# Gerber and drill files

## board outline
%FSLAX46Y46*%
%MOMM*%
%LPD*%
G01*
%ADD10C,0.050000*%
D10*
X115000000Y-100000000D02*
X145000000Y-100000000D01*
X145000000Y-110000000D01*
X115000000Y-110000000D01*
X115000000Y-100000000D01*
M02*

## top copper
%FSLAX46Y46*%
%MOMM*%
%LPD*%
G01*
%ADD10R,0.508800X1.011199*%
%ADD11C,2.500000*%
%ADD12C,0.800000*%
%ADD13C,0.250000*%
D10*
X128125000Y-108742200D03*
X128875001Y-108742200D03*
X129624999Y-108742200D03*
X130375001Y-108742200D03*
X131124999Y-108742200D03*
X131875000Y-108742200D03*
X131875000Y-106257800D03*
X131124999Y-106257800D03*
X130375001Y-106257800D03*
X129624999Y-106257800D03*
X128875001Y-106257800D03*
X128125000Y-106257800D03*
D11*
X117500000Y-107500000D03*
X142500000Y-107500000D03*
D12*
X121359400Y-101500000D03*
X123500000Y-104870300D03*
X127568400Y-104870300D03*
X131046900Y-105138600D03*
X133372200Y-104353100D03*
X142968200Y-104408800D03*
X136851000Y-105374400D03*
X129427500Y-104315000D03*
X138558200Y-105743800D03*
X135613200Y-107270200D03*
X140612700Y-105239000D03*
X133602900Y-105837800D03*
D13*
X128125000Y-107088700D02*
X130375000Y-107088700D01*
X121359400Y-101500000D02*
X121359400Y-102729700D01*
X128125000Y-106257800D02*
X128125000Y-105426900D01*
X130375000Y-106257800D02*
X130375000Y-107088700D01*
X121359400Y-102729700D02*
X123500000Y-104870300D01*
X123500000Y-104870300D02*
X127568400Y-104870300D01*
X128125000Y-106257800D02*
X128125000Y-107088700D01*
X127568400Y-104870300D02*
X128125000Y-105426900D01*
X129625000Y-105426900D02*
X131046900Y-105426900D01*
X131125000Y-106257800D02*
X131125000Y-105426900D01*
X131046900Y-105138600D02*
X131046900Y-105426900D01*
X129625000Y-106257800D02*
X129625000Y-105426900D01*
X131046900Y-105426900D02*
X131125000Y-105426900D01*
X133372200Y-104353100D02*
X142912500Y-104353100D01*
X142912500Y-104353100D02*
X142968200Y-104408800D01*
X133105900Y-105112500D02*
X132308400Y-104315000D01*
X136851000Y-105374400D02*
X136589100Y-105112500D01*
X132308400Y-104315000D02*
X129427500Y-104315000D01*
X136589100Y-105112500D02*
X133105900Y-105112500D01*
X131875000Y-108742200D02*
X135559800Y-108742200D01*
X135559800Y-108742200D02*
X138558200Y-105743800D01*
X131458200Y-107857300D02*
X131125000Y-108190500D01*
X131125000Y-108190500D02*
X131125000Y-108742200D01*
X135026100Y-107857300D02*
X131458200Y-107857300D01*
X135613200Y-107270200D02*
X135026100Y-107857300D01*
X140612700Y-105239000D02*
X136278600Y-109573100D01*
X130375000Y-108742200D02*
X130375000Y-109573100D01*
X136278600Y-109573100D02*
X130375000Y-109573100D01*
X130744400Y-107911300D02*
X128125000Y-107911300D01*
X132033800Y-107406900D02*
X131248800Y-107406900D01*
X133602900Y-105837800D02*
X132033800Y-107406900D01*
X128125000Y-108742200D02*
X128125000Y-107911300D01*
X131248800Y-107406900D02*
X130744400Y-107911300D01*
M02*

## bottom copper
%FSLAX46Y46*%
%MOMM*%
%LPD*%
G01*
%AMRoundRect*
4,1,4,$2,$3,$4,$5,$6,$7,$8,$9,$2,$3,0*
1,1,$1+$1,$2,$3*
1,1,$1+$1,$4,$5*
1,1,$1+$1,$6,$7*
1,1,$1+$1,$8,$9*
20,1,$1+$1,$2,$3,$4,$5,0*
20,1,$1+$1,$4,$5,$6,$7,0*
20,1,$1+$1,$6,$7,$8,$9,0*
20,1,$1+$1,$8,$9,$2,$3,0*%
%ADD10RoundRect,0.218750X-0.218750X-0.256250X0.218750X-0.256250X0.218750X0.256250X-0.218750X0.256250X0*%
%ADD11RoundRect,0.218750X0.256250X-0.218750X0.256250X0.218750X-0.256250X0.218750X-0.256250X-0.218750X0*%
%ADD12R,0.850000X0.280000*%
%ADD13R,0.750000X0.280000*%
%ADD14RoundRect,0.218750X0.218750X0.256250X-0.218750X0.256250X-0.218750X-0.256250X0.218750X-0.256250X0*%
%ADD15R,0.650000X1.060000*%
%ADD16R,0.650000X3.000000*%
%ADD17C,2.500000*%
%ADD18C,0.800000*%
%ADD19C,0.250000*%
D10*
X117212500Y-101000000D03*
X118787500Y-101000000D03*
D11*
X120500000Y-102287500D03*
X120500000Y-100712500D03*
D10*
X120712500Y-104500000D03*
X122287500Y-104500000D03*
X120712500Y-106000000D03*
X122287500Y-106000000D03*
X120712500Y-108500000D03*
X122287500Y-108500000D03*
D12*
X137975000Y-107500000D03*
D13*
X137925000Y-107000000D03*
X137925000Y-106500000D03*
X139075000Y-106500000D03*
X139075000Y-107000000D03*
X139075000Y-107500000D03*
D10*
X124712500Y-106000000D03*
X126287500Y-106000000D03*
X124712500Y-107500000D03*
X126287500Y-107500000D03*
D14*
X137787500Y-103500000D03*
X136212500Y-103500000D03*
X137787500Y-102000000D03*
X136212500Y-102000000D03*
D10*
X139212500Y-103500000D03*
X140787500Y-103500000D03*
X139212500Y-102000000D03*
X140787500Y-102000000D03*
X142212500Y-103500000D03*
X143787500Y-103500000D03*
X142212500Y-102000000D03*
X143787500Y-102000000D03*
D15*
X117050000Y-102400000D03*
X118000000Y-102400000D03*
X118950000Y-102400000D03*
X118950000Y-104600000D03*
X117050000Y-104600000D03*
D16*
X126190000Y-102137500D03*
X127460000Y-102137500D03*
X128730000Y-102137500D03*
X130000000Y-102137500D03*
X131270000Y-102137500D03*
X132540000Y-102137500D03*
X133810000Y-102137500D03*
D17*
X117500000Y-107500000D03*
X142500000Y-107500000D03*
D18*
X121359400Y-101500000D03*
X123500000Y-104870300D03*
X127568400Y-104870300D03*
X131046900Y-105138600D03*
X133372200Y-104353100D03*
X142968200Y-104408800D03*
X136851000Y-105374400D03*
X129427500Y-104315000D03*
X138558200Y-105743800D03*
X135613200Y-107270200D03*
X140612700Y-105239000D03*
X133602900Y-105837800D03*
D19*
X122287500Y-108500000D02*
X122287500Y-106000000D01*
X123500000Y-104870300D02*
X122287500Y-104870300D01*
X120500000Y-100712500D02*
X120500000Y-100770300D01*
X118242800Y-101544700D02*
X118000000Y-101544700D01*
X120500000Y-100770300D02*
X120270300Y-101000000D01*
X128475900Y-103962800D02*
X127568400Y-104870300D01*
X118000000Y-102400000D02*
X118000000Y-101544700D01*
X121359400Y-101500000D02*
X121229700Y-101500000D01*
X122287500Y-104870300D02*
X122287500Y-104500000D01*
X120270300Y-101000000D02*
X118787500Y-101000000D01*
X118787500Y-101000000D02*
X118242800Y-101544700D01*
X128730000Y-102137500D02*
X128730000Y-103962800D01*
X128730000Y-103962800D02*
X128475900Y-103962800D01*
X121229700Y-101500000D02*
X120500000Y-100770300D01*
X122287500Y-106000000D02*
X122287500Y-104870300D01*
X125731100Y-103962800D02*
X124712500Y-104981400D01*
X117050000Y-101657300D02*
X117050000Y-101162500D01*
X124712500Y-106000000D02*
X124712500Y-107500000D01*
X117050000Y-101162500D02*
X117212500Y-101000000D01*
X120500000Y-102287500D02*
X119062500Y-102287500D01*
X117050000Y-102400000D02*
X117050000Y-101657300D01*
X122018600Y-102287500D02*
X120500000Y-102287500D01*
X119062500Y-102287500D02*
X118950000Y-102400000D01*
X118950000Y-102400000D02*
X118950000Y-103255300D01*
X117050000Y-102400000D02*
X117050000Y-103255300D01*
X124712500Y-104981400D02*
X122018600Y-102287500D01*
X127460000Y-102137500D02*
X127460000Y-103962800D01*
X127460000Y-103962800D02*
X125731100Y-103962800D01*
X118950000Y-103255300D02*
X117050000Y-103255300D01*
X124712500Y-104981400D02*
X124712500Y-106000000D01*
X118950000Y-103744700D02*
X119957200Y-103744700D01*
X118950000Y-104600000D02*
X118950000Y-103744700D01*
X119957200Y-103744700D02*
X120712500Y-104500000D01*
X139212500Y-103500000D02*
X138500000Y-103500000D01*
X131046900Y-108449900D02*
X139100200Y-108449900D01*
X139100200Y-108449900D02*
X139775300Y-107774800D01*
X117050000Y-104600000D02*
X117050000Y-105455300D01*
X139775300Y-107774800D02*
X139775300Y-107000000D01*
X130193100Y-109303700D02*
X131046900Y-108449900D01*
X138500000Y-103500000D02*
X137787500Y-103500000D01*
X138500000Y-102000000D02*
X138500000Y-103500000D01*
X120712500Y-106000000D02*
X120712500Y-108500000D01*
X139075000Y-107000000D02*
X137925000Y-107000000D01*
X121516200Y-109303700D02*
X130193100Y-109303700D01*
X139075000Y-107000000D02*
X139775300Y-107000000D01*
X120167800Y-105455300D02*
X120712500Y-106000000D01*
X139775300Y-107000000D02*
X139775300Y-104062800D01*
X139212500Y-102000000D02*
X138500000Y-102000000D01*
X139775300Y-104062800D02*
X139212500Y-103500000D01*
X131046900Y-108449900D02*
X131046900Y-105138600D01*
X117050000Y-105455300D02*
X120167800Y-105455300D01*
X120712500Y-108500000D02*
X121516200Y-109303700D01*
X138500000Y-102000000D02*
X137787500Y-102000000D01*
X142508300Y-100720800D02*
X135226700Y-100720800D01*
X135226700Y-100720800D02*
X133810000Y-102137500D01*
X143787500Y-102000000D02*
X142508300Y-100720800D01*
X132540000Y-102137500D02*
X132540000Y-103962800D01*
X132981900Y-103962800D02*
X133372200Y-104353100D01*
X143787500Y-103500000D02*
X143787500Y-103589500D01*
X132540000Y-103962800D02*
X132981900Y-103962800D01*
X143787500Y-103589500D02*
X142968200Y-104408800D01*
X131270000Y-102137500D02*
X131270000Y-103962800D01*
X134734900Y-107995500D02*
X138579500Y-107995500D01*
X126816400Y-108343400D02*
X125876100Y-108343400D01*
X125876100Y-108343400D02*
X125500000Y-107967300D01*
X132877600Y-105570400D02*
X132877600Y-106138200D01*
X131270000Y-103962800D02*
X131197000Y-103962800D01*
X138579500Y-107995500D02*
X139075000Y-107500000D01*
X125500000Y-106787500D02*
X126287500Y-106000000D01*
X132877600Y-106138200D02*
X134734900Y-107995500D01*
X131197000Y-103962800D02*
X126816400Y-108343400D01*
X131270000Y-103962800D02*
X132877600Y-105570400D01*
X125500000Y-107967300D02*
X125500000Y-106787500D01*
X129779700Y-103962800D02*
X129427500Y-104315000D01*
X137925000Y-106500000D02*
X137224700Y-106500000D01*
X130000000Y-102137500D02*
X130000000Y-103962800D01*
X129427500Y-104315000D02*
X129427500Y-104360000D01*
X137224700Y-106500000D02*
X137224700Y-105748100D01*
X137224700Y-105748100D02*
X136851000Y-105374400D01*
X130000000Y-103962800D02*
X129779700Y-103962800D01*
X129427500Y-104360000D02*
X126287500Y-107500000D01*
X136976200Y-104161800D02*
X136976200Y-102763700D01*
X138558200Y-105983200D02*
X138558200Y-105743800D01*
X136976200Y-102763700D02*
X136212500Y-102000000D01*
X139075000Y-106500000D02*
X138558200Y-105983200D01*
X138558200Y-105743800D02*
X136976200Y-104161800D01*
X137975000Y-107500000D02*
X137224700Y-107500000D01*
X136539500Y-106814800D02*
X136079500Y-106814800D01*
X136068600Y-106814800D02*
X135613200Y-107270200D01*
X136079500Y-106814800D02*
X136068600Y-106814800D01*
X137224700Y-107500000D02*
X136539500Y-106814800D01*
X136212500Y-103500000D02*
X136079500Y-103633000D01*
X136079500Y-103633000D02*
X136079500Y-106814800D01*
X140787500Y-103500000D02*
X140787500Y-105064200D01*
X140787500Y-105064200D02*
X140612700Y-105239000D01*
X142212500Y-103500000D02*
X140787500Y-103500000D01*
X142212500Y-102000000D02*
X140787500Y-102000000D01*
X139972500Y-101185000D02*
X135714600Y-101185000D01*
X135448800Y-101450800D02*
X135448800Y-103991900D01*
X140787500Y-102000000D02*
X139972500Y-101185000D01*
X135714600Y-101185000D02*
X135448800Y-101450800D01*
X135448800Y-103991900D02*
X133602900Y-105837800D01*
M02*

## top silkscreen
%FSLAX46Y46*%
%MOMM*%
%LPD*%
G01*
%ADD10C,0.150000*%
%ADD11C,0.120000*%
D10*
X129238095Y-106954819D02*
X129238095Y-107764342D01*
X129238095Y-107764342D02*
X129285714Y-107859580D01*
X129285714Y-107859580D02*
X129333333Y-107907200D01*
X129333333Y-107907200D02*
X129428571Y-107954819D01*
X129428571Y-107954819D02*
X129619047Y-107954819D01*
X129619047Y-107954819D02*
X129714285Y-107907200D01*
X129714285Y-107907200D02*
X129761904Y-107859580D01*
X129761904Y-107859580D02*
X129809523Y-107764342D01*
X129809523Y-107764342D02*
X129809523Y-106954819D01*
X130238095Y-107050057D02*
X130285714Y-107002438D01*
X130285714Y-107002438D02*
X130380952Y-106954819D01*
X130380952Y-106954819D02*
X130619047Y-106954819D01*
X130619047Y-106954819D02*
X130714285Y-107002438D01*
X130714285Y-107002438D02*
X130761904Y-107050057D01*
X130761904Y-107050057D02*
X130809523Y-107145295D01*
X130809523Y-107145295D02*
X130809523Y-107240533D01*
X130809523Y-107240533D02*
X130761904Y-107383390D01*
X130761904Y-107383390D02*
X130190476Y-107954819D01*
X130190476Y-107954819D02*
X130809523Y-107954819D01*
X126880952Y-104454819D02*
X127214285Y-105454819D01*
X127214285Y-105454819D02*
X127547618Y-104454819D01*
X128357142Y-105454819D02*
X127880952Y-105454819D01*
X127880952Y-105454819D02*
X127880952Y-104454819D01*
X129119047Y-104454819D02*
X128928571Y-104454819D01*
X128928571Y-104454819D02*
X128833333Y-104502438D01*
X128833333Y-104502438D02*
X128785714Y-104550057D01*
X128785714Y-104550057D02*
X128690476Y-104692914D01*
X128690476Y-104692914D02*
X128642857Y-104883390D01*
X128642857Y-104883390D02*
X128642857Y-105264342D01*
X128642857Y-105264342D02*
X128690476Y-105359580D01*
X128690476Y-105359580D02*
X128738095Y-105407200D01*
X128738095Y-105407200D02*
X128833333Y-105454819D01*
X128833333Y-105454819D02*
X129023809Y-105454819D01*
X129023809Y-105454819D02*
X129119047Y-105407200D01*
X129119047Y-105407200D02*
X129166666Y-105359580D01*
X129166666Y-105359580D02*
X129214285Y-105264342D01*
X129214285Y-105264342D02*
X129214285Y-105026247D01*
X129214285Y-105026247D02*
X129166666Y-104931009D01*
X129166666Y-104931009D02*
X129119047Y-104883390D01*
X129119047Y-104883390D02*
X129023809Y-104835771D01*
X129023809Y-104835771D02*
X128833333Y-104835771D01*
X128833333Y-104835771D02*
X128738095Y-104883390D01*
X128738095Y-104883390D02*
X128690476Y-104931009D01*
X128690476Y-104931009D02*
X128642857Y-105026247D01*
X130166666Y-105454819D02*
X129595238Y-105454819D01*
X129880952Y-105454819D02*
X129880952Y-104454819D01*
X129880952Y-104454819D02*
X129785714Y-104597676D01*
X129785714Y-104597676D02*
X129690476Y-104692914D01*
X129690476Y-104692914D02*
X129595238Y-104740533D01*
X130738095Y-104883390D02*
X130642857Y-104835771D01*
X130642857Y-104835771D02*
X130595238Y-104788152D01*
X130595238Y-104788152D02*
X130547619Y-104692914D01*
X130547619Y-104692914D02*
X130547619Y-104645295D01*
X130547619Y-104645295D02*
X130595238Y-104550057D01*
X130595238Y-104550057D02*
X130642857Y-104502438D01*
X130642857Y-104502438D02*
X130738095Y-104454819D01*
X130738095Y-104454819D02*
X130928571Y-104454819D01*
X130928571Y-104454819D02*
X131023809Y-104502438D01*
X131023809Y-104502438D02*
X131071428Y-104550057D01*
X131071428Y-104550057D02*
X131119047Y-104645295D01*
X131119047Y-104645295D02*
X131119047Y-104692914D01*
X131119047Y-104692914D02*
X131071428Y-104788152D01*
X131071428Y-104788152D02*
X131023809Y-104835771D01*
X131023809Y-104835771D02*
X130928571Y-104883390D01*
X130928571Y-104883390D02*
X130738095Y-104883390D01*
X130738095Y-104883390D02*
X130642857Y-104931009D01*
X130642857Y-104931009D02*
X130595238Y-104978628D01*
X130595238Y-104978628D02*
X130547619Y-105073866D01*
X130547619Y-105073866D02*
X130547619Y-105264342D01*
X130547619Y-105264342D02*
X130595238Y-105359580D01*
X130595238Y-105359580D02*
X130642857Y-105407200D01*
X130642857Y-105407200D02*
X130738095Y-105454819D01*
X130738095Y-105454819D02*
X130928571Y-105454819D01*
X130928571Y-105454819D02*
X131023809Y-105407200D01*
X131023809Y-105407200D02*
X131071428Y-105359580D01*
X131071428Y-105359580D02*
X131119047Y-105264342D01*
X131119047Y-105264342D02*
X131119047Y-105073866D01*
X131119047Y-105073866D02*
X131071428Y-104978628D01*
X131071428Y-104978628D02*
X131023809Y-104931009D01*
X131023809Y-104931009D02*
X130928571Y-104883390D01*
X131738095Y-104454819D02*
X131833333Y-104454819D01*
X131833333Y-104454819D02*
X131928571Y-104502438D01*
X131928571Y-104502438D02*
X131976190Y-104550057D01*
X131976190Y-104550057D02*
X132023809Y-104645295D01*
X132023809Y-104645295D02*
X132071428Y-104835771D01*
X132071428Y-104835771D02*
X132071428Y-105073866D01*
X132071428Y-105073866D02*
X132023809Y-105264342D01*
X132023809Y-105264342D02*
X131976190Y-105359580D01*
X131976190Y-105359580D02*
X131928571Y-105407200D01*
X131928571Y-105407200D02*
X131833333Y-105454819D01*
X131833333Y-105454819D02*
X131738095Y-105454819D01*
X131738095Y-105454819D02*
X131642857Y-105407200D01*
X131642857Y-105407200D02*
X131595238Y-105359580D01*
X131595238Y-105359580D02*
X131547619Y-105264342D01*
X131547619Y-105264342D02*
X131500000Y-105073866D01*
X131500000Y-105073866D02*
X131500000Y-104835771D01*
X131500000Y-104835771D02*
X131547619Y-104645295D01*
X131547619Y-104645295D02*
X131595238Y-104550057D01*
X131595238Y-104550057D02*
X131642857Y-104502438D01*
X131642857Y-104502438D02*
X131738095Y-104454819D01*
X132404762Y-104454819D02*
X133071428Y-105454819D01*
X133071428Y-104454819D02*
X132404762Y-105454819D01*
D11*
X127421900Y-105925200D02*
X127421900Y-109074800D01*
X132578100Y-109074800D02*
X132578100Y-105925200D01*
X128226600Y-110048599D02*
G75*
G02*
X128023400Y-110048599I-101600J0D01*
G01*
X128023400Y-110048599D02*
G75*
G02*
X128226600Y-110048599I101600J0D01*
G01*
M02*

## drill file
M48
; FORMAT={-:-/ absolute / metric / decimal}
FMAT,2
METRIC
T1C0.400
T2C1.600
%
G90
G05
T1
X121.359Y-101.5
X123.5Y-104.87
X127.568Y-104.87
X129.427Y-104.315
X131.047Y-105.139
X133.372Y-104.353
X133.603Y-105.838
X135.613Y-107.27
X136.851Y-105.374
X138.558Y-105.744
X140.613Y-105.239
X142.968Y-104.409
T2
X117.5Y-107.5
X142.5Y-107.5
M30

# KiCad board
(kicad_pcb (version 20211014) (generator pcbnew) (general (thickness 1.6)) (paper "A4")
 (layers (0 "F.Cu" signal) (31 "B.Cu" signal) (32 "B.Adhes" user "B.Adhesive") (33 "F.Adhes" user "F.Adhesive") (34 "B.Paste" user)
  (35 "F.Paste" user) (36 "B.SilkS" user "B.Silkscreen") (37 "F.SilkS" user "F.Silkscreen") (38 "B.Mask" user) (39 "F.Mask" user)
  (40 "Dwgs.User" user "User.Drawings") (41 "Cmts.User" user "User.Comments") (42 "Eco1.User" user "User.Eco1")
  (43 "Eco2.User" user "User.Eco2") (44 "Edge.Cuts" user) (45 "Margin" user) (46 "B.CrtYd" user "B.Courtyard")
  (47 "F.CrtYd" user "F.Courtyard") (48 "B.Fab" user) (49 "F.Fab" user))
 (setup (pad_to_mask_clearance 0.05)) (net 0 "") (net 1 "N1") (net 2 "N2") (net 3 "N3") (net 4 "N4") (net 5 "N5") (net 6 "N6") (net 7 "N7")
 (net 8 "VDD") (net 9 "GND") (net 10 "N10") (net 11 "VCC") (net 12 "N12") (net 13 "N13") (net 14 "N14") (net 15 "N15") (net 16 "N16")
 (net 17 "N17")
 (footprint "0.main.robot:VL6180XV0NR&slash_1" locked (layer "F.Cu") (at 130 107.5 90)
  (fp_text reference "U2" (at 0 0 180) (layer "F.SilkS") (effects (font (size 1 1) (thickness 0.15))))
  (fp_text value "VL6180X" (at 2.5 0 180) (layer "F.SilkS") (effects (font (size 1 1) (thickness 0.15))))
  (fp_line (start 1.5748 -2.5781) (end -1.5748 -2.5781) (layer "F.SilkS") (width 0.12))
  (fp_line (start -1.5748 2.5781) (end 1.5748 2.5781) (layer "F.SilkS") (width 0.12))
  (fp_circle (center -2.548599 -1.875) (end -2.446999 -1.875) (layer "F.SilkS") (width 0.12) (fill none))
  (pad "1" smd rect locked (at -1.2422 -1.875 90) (size 1.011199 0.5088) (layers "F.Cu" "F.Paste" "F.Mask") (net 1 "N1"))
  (pad "2" smd rect locked (at -1.2422 -1.124999 90) (size 1.011199 0.5088) (layers "F.Cu" "F.Paste" "F.Mask") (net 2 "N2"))
  (pad "3" smd rect locked (at -1.2422 -0.375001 90) (size 1.011199 0.5088) (layers "F.Cu" "F.Paste" "F.Mask") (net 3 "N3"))
  (pad "4" smd rect locked (at -1.2422 0.375001 90) (size 1.011199 0.5088) (layers "F.Cu" "F.Paste" "F.Mask") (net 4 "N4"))
  (pad "5" smd rect locked (at -1.2422 1.124999 90) (size 1.011199 0.5088) (layers "F.Cu" "F.Paste" "F.Mask") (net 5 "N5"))
  (pad "6" smd rect locked (at -1.2422 1.875 90) (size 1.011199 0.5088) (layers "F.Cu" "F.Paste" "F.Mask") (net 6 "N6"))
  (pad "7" smd rect locked (at 1.2422 1.875 90) (size 1.011199 0.5088) (layers "F.Cu" "F.Paste" "F.Mask") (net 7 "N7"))
  (pad "8" smd rect locked (at 1.2422 1.124999 90) (size 1.011199 0.5088) (layers "F.Cu" "F.Paste" "F.Mask") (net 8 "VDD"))
  (pad "9" smd rect locked (at 1.2422 0.375001 90) (size 1.011199 0.5088) (layers "F.Cu" "F.Paste" "F.Mask") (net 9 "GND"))
  (pad "10" smd rect locked (at 1.2422 -0.375001 90) (size 1.011199 0.5088) (layers "F.Cu" "F.Paste" "F.Mask") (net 8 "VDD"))
  (pad "11" smd rect locked (at 1.2422 -1.124999 90) (size 1.011199 0.5088) (layers "F.Cu" "F.Paste" "F.Mask") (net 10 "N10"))
  (pad "12" smd rect locked (at 1.2422 -1.875 90) (size 1.011199 0.5088) (layers "F.Cu" "F.Paste" "F.Mask") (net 9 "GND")))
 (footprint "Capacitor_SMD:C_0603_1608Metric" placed (layer "B.Cu") (at 118 101)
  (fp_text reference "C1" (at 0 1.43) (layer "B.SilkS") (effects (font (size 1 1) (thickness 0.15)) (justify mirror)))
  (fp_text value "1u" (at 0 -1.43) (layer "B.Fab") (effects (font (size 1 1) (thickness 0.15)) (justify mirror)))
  (pad "1" smd roundrect locked (at -0.7875 0) (size 0.875 0.95) (layers "B.Cu" "B.Paste" "B.Mask") (roundrect_rratio 0.25) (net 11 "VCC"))
  (pad "2" smd roundrect locked (at 0.7875 0) (size 0.875 0.95) (layers "B.Cu" "B.Paste" "B.Mask") (roundrect_rratio 0.25) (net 9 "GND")))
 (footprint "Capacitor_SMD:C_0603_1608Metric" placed (layer "B.Cu") (at 120.5 101.5 90)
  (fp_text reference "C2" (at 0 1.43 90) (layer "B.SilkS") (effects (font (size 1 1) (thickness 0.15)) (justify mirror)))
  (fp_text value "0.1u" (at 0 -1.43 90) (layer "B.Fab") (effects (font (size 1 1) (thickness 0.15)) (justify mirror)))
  (pad "1" smd roundrect locked (at -0.7875 0 90) (size 0.875 0.95) (layers "B.Cu" "B.Paste" "B.Mask") (roundrect_rratio 0.25)
   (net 11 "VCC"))
  (pad "2" smd roundrect locked (at 0.7875 0 90) (size 0.875 0.95) (layers "B.Cu" "B.Paste" "B.Mask") (roundrect_rratio 0.25) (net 9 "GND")))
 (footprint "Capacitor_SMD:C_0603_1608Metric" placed (layer "B.Cu") (at 121.5 104.5)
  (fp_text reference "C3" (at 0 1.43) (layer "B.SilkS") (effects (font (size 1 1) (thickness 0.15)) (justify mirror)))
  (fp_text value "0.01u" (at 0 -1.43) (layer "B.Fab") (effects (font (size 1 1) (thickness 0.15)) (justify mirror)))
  (pad "1" smd roundrect locked (at -0.7875 0) (size 0.875 0.95) (layers "B.Cu" "B.Paste" "B.Mask") (roundrect_rratio 0.25) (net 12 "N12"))
  (pad "2" smd roundrect locked (at 0.7875 0) (size 0.875 0.95) (layers "B.Cu" "B.Paste" "B.Mask") (roundrect_rratio 0.25) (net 9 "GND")))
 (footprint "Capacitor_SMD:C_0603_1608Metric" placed (layer "B.Cu") (at 121.5 106)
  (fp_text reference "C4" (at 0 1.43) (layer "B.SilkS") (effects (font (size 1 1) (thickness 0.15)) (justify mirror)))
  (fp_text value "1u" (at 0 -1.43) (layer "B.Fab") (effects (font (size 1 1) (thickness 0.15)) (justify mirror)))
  (pad "1" smd roundrect locked (at -0.7875 0) (size 0.875 0.95) (layers "B.Cu" "B.Paste" "B.Mask") (roundrect_rratio 0.25) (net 8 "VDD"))
  (pad "2" smd roundrect locked (at 0.7875 0) (size 0.875 0.95) (layers "B.Cu" "B.Paste" "B.Mask") (roundrect_rratio 0.25) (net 9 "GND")))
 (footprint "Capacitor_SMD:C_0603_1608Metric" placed (layer "B.Cu") (at 121.5 108.5)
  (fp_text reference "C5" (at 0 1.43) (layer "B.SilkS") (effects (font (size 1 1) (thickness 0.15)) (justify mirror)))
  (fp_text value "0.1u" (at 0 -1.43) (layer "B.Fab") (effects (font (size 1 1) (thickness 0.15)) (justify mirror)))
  (pad "1" smd roundrect locked (at -0.7875 0) (size 0.875 0.95) (layers "B.Cu" "B.Paste" "B.Mask") (roundrect_rratio 0.25) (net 8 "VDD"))
  (pad "2" smd roundrect locked (at 0.7875 0) (size 0.875 0.95) (layers "B.Cu" "B.Paste" "B.Mask") (roundrect_rratio 0.25) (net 9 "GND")))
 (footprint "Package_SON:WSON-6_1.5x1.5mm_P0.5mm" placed (layer "B.Cu") (at 138.5 107)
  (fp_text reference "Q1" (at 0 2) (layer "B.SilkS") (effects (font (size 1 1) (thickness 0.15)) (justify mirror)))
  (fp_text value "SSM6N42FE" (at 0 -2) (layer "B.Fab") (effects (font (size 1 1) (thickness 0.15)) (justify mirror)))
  (pad "1" smd rect locked (at -0.525 0.5 90) (size 0.28 0.85) (layers "B.Cu" "B.Paste" "B.Mask") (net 5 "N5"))
  (pad "2" smd rect locked (at -0.575 0 90) (size 0.28 0.75) (layers "B.Cu" "B.Paste" "B.Mask") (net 8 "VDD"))
  (pad "3" smd rect locked (at -0.575 -0.5 90) (size 0.28 0.75) (layers "B.Cu" "B.Paste" "B.Mask") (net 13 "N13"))
  (pad "4" smd rect locked (at 0.575 -0.5 90) (size 0.28 0.75) (layers "B.Cu" "B.Paste" "B.Mask") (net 6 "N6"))
  (pad "5" smd rect locked (at 0.575 0 90) (size 0.28 0.75) (layers "B.Cu" "B.Paste" "B.Mask") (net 8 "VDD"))
  (pad "6" smd rect locked (at 0.575 0.5 90) (size 0.28 0.75) (layers "B.Cu" "B.Paste" "B.Mask") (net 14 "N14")))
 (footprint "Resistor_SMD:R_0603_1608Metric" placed (layer "B.Cu") (at 125.5 106)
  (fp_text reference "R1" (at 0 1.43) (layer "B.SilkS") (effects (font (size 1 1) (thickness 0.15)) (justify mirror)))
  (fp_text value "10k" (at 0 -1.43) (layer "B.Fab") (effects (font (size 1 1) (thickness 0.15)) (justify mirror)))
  (pad "1" smd roundrect locked (at -0.7875 0) (size 0.875 0.95) (layers "B.Cu" "B.Paste" "B.Mask") (roundrect_rratio 0.25) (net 11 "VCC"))
  (pad "2" smd roundrect locked (at 0.7875 0) (size 0.875 0.95) (layers "B.Cu" "B.Paste" "B.Mask") (roundrect_rratio 0.25) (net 14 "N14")))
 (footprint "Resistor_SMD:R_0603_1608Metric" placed (layer "B.Cu") (at 125.5 107.5)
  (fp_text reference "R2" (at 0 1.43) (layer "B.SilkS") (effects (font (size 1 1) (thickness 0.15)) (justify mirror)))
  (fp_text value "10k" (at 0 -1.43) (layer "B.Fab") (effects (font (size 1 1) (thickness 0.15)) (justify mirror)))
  (pad "1" smd roundrect locked (at -0.7875 0) (size 0.875 0.95) (layers "B.Cu" "B.Paste" "B.Mask") (roundrect_rratio 0.25) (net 11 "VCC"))
  (pad "2" smd roundrect locked (at 0.7875 0) (size 0.875 0.95) (layers "B.Cu" "B.Paste" "B.Mask") (roundrect_rratio 0.25) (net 13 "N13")))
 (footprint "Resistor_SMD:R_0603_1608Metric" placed (layer "B.Cu") (at 137 103.5 180)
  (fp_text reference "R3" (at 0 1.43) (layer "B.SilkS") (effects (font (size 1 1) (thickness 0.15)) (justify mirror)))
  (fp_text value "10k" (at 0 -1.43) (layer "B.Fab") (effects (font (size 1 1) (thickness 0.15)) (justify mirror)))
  (pad "1" smd roundrect locked (at -0.7875 0 180) (size 0.875 0.95) (layers "B.Cu" "B.Paste" "B.Mask") (roundrect_rratio 0.25)
   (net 8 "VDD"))
  (pad "2" smd roundrect locked (at 0.7875 0 180) (size 0.875 0.95) (layers "B.Cu" "B.Paste" "B.Mask") (roundrect_rratio 0.25) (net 5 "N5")))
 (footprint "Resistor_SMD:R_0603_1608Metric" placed (layer "B.Cu") (at 137 102 180)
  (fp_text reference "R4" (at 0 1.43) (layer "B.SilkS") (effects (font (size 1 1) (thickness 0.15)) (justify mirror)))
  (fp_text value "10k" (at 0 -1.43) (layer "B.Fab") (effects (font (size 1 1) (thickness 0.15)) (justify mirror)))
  (pad "1" smd roundrect locked (at -0.7875 0 180) (size 0.875 0.95) (layers "B.Cu" "B.Paste" "B.Mask") (roundrect_rratio 0.25)
   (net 8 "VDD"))
  (pad "2" smd roundrect locked (at 0.7875 0 180) (size 0.875 0.95) (layers "B.Cu" "B.Paste" "B.Mask") (roundrect_rratio 0.25) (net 6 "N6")))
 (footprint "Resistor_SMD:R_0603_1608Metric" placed (layer "B.Cu") (at 140 103.5)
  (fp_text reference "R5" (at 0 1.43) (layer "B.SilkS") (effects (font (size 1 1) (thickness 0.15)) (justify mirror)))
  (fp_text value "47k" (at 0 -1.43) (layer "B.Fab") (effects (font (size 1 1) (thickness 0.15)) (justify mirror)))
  (pad "1" smd roundrect locked (at -0.7875 0) (size 0.875 0.95) (layers "B.Cu" "B.Paste" "B.Mask") (roundrect_rratio 0.25) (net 8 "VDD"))
  (pad "2" smd roundrect locked (at 0.7875 0) (size 0.875 0.95) (layers "B.Cu" "B.Paste" "B.Mask") (roundrect_rratio 0.25) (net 4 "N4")))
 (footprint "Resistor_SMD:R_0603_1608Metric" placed (layer "B.Cu") (at 140 102)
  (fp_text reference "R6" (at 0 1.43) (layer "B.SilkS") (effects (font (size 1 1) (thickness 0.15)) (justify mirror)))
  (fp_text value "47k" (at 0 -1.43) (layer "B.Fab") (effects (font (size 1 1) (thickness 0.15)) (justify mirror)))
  (pad "1" smd roundrect locked (at -0.7875 0) (size 0.875 0.95) (layers "B.Cu" "B.Paste" "B.Mask") (roundrect_rratio 0.25) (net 8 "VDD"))
  (pad "2" smd roundrect locked (at 0.7875 0) (size 0.875 0.95) (layers "B.Cu" "B.Paste" "B.Mask") (roundrect_rratio 0.25) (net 1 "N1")))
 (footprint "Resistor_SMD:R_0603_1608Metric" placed (layer "B.Cu") (at 143 103.5)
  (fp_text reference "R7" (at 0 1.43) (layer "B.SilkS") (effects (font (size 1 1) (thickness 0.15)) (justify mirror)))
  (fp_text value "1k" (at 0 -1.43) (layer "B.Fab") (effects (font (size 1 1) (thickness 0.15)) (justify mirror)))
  (pad "1" smd roundrect locked (at -0.7875 0) (size 0.875 0.95) (layers "B.Cu" "B.Paste" "B.Mask") (roundrect_rratio 0.25) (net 4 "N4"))
  (pad "2" smd roundrect locked (at 0.7875 0) (size 0.875 0.95) (layers "B.Cu" "B.Paste" "B.Mask") (roundrect_rratio 0.25) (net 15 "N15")))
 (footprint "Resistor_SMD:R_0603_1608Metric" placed (layer "B.Cu") (at 143 102)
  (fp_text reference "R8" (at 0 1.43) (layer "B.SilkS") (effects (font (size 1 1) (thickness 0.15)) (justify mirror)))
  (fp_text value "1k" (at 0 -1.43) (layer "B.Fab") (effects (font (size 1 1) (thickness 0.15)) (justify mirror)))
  (pad "1" smd roundrect locked (at -0.7875 0) (size 0.875 0.95) (layers "B.Cu" "B.Paste" "B.Mask") (roundrect_rratio 0.25) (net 1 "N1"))
  (pad "2" smd roundrect locked (at 0.7875 0) (size 0.875 0.95) (layers "B.Cu" "B.Paste" "B.Mask") (roundrect_rratio 0.25) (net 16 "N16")))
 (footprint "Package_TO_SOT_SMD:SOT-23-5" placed (layer "B.Cu") (at 118 103.5 -90)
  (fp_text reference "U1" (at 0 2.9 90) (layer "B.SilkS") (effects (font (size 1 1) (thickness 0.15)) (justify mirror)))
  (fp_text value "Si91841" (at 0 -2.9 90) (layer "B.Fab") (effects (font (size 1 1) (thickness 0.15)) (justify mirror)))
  (pad "1" smd rect locked (at -1.1 0.95 270) (size 1.06 0.65) (layers "B.Cu" "B.Paste" "B.Mask") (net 11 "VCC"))
  (pad "2" smd rect locked (at -1.1 0 270) (size 1.06 0.65) (layers "B.Cu" "B.Paste" "B.Mask") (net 9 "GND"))
  (pad "3" smd rect locked (at -1.1 -0.95 270) (size 1.06 0.65) (layers "B.Cu" "B.Paste" "B.Mask") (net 11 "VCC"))
  (pad "4" smd rect locked (at 1.1 -0.95 270) (size 1.06 0.65) (layers "B.Cu" "B.Paste" "B.Mask") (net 12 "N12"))
  (pad "5" smd rect locked (at 1.1 0.95 270) (size 1.06 0.65) (layers "B.Cu" "B.Paste" "B.Mask") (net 8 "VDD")))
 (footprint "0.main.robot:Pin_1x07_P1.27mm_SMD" (layer "B.Cu") (at 130 103.6375 -90)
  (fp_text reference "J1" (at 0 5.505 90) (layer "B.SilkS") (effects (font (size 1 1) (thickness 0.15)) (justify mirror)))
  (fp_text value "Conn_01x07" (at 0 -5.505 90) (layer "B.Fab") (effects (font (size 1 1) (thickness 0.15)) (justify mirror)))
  (pad "1" smd rect (at -1.5 3.81 270) (size 3 0.65) (layers "B.Cu" "B.Paste" "B.Mask") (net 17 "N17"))
  (pad "2" smd rect (at -1.5 2.54 270) (size 3 0.65) (layers "B.Cu" "B.Paste" "B.Mask") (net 11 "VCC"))
  (pad "3" smd rect (at -1.5 1.27 270) (size 3 0.65) (layers "B.Cu" "B.Paste" "B.Mask") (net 9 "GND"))
  (pad "4" smd rect (at -1.5 0 270) (size 3 0.65) (layers "B.Cu" "B.Paste" "B.Mask") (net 13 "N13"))
  (pad "5" smd rect (at -1.5 -1.27 270) (size 3 0.65) (layers "B.Cu" "B.Paste" "B.Mask") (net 14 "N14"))
  (pad "6" smd rect (at -1.5 -2.54 270) (size 3 0.65) (layers "B.Cu" "B.Paste" "B.Mask") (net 15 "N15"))
  (pad "7" smd rect (at -1.5 -3.81 270) (size 3 0.65) (layers "B.Cu" "B.Paste" "B.Mask") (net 16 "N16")))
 (gr_rect (start 115 100) (end 145 110) (layer "Edge.Cuts") (width 0.05) (fill none))
 (via (at 117.5 107.5) (size 2.5) (drill 1.6) (layers "F.Cu" "B.Cu") (free) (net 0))
 (via (at 142.5 107.5) (size 2.5) (drill 1.6) (layers "F.Cu" "B.Cu") (free) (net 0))
 (segment (start 128.125 107.0887) (end 130.375 107.0887) (width 0.25) (layer "F.Cu") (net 9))
 (segment (start 121.3594 101.5) (end 121.3594 102.7297) (width 0.25) (layer "F.Cu") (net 9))
 (segment (start 128.125 106.2578) (end 128.125 105.4269) (width 0.25) (layer "F.Cu") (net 9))
 (segment (start 130.375 106.2578) (end 130.375 107.0887) (width 0.25) (layer "F.Cu") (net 9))
 (segment (start 121.3594 102.7297) (end 123.5 104.8703) (width 0.25) (layer "F.Cu") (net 9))
 (segment (start 123.5 104.8703) (end 127.5684 104.8703) (width 0.25) (layer "F.Cu") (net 9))
 (segment (start 128.125 106.2578) (end 128.125 107.0887) (width 0.25) (layer "F.Cu") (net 9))
 (segment (start 127.5684 104.8703) (end 128.125 105.4269) (width 0.25) (layer "F.Cu") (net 9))
 (via (at 121.3594 101.5) (size 0.8) (drill 0.4) (layers "F.Cu" "B.Cu") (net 9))
 (via (at 123.5 104.8703) (size 0.8) (drill 0.4) (layers "F.Cu" "B.Cu") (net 9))
 (via (at 127.5684 104.8703) (size 0.8) (drill 0.4) (layers "F.Cu" "B.Cu") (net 9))
 (segment (start 122.2875 108.5) (end 122.2875 106) (width 0.25) (layer "B.Cu") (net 9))
 (segment (start 123.5 104.8703) (end 122.2875 104.8703) (width 0.25) (layer "B.Cu") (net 9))
 (segment (start 120.5 100.7125) (end 120.5 100.7703) (width 0.25) (layer "B.Cu") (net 9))
 (segment (start 118.2428 101.5447) (end 118 101.5447) (width 0.25) (layer "B.Cu") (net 9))
 (segment (start 120.5 100.7703) (end 120.2703 101) (width 0.25) (layer "B.Cu") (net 9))
 (segment (start 128.4759 103.9628) (end 127.5684 104.8703) (width 0.25) (layer "B.Cu") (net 9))
 (segment (start 118 102.4) (end 118 101.5447) (width 0.25) (layer "B.Cu") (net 9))
 (segment (start 121.3594 101.5) (end 121.2297 101.5) (width 0.25) (layer "B.Cu") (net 9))
 (segment (start 122.2875 104.8703) (end 122.2875 104.5) (width 0.25) (layer "B.Cu") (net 9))
 (segment (start 120.2703 101) (end 118.7875 101) (width 0.25) (layer "B.Cu") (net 9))
 (segment (start 118.7875 101) (end 118.2428 101.5447) (width 0.25) (layer "B.Cu") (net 9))
 (segment (start 128.73 102.1375) (end 128.73 103.9628) (width 0.25) (layer "B.Cu") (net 9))
 (segment (start 128.73 103.9628) (end 128.4759 103.9628) (width 0.25) (layer "B.Cu") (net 9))
 (segment (start 121.2297 101.5) (end 120.5 100.7703) (width 0.25) (layer "B.Cu") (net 9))
 (segment (start 122.2875 106) (end 122.2875 104.8703) (width 0.25) (layer "B.Cu") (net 9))
 (segment (start 125.7311 103.9628) (end 124.7125 104.9814) (width 0.25) (layer "B.Cu") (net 11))
 (segment (start 117.05 101.6573) (end 117.05 101.1625) (width 0.25) (layer "B.Cu") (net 11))
 (segment (start 124.7125 106) (end 124.7125 107.5) (width 0.25) (layer "B.Cu") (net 11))
 (segment (start 117.05 101.1625) (end 117.2125 101) (width 0.25) (layer "B.Cu") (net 11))
 (segment (start 120.5 102.2875) (end 119.0625 102.2875) (width 0.25) (layer "B.Cu") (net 11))
 (segment (start 117.05 102.4) (end 117.05 101.6573) (width 0.25) (layer "B.Cu") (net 11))
 (segment (start 122.0186 102.2875) (end 120.5 102.2875) (width 0.25) (layer "B.Cu") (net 11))
 (segment (start 119.0625 102.2875) (end 118.95 102.4) (width 0.25) (layer "B.Cu") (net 11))
 (segment (start 118.95 102.4) (end 118.95 103.2553) (width 0.25) (layer "B.Cu") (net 11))
 (segment (start 117.05 102.4) (end 117.05 103.2553) (width 0.25) (layer "B.Cu") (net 11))
 (segment (start 124.7125 104.9814) (end 122.0186 102.2875) (width 0.25) (layer "B.Cu") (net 11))
 (segment (start 127.46 102.1375) (end 127.46 103.9628) (width 0.25) (layer "B.Cu") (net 11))
 (segment (start 127.46 103.9628) (end 125.7311 103.9628) (width 0.25) (layer "B.Cu") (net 11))
 (segment (start 118.95 103.2553) (end 117.05 103.2553) (width 0.25) (layer "B.Cu") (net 11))
 (segment (start 124.7125 104.9814) (end 124.7125 106) (width 0.25) (layer "B.Cu") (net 11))
 (segment (start 118.95 103.7447) (end 119.9572 103.7447) (width 0.25) (layer "B.Cu") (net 12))
 (segment (start 118.95 104.6) (end 118.95 103.7447) (width 0.25) (layer "B.Cu") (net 12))
 (segment (start 119.9572 103.7447) (end 120.7125 104.5) (width 0.25) (layer "B.Cu") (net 12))
 (segment (start 129.625 105.4269) (end 131.0469 105.4269) (width 0.25) (layer "F.Cu") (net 8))
 (segment (start 131.125 106.2578) (end 131.125 105.4269) (width 0.25) (layer "F.Cu") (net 8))
 (segment (start 131.0469 105.1386) (end 131.0469 105.4269) (width 0.25) (layer "F.Cu") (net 8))
 (segment (start 129.625 106.2578) (end 129.625 105.4269) (width 0.25) (layer "F.Cu") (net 8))
 (segment (start 131.0469 105.4269) (end 131.125 105.4269) (width 0.25) (layer "F.Cu") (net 8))
 (via (at 131.0469 105.1386) (size 0.8) (drill 0.4) (layers "F.Cu" "B.Cu") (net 8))
 (segment (start 139.2125 103.5) (end 138.5 103.5) (width 0.25) (layer "B.Cu") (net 8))
 (segment (start 131.0469 108.4499) (end 139.1002 108.4499) (width 0.25) (layer "B.Cu") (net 8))
 (segment (start 139.1002 108.4499) (end 139.7753 107.7748) (width 0.25) (layer "B.Cu") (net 8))
 (segment (start 117.05 104.6) (end 117.05 105.4553) (width 0.25) (layer "B.Cu") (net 8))
 (segment (start 139.7753 107.7748) (end 139.7753 107) (width 0.25) (layer "B.Cu") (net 8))
 (segment (start 130.1931 109.3037) (end 131.0469 108.4499) (width 0.25) (layer "B.Cu") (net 8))
 (segment (start 138.5 103.5) (end 137.7875 103.5) (width 0.25) (layer "B.Cu") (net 8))
 (segment (start 138.5 102) (end 138.5 103.5) (width 0.25) (layer "B.Cu") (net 8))
 (segment (start 120.7125 106) (end 120.7125 108.5) (width 0.25) (layer "B.Cu") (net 8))
 (segment (start 139.075 107) (end 137.925 107) (width 0.25) (layer "B.Cu") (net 8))
 (segment (start 121.5162 109.3037) (end 130.1931 109.3037) (width 0.25) (layer "B.Cu") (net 8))
 (segment (start 139.075 107) (end 139.7753 107) (width 0.25) (layer "B.Cu") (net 8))
 (segment (start 120.1678 105.4553) (end 120.7125 106) (width 0.25) (layer "B.Cu") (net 8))
 (segment (start 139.7753 107) (end 139.7753 104.0628) (width 0.25) (layer "B.Cu") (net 8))
 (segment (start 139.2125 102) (end 138.5 102) (width 0.25) (layer "B.Cu") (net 8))
 (segment (start 139.7753 104.0628) (end 139.2125 103.5) (width 0.25) (layer "B.Cu") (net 8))
 (segment (start 131.0469 108.4499) (end 131.0469 105.1386) (width 0.25) (layer "B.Cu") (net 8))
 (segment (start 117.05 105.4553) (end 120.1678 105.4553) (width 0.25) (layer "B.Cu") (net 8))
 (segment (start 120.7125 108.5) (end 121.5162 109.3037) (width 0.25) (layer "B.Cu") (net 8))
 (segment (start 138.5 102) (end 137.7875 102) (width 0.25) (layer "B.Cu") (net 8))
 (segment (start 142.5083 100.7208) (end 135.2267 100.7208) (width 0.25) (layer "B.Cu") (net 16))
 (segment (start 135.2267 100.7208) (end 133.81 102.1375) (width 0.25) (layer "B.Cu") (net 16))
 (segment (start 143.7875 102) (end 142.5083 100.7208) (width 0.25) (layer "B.Cu") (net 16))
 (segment (start 133.3722 104.3531) (end 142.9125 104.3531) (width 0.25) (layer "F.Cu") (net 15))
 (segment (start 142.9125 104.3531) (end 142.9682 104.4088) (width 0.25) (layer "F.Cu") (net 15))
 (via (at 133.3722 104.3531) (size 0.8) (drill 0.4) (layers "F.Cu" "B.Cu") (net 15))
 (via (at 142.9682 104.4088) (size 0.8) (drill 0.4) (layers "F.Cu" "B.Cu") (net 15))
 (segment (start 132.54 102.1375) (end 132.54 103.9628) (width 0.25) (layer "B.Cu") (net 15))
 (segment (start 132.9819 103.9628) (end 133.3722 104.3531) (width 0.25) (layer "B.Cu") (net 15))
 (segment (start 143.7875 103.5) (end 143.7875 103.5895) (width 0.25) (layer "B.Cu") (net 15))
 (segment (start 132.54 103.9628) (end 132.9819 103.9628) (width 0.25) (layer "B.Cu") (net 15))
 (segment (start 143.7875 103.5895) (end 142.9682 104.4088) (width 0.25) (layer "B.Cu") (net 15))
 (segment (start 131.27 102.1375) (end 131.27 103.9628) (width 0.25) (layer "B.Cu") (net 14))
 (segment (start 134.7349 107.9955) (end 138.5795 107.9955) (width 0.25) (layer "B.Cu") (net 14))
 (segment (start 126.8164 108.3434) (end 125.8761 108.3434) (width 0.25) (layer "B.Cu") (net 14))
 (segment (start 125.8761 108.3434) (end 125.5 107.9673) (width 0.25) (layer "B.Cu") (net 14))
 (segment (start 132.8776 105.5704) (end 132.8776 106.1382) (width 0.25) (layer "B.Cu") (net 14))
 (segment (start 131.27 103.9628) (end 131.197 103.9628) (width 0.25) (layer "B.Cu") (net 14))
 (segment (start 138.5795 107.9955) (end 139.075 107.5) (width 0.25) (layer "B.Cu") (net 14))
 (segment (start 125.5 106.7875) (end 126.2875 106) (width 0.25) (layer "B.Cu") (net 14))
 (segment (start 132.8776 106.1382) (end 134.7349 107.9955) (width 0.25) (layer "B.Cu") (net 14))
 (segment (start 131.197 103.9628) (end 126.8164 108.3434) (width 0.25) (layer "B.Cu") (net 14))
 (segment (start 131.27 103.9628) (end 132.8776 105.5704) (width 0.25) (layer "B.Cu") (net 14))
 (segment (start 125.5 107.9673) (end 125.5 106.7875) (width 0.25) (layer "B.Cu") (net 14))
 (segment (start 133.1059 105.1125) (end 132.3084 104.315) (width 0.25) (layer "F.Cu") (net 13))
 (segment (start 136.851 105.3744) (end 136.5891 105.1125) (width 0.25) (layer "F.Cu") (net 13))
 (segment (start 132.3084 104.315) (end 129.4275 104.315) (width 0.25) (layer "F.Cu") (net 13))
 (segment (start 136.5891 105.1125) (end 133.1059 105.1125) (width 0.25) (layer "F.Cu") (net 13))
 (via (at 136.851 105.3744) (size 0.8) (drill 0.4) (layers "F.Cu" "B.Cu") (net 13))
 (via (at 129.4275 104.315) (size 0.8) (drill 0.4) (layers "F.Cu" "B.Cu") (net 13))
 (segment (start 129.7797 103.9628) (end 129.4275 104.315) (width 0.25) (layer "B.Cu") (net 13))
 (segment (start 137.925 106.5) (end 137.2247 106.5) (width 0.25) (layer "B.Cu") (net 13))
 (segment (start 130 102.1375) (end 130 103.9628) (width 0.25) (layer "B.Cu") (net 13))
 (segment (start 129.4275 104.315) (end 129.4275 104.36) (width 0.25) (layer "B.Cu") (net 13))
 (segment (start 137.2247 106.5) (end 137.2247 105.7481) (width 0.25) (layer "B.Cu") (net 13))
 (segment (start 137.2247 105.7481) (end 136.851 105.3744) (width 0.25) (layer "B.Cu") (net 13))
 (segment (start 130 103.9628) (end 129.7797 103.9628) (width 0.25) (layer "B.Cu") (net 13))
 (segment (start 129.4275 104.36) (end 126.2875 107.5) (width 0.25) (layer "B.Cu") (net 13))
 (segment (start 131.875 108.7422) (end 135.5598 108.7422) (width 0.25) (layer "F.Cu") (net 6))
 (segment (start 135.5598 108.7422) (end 138.5582 105.7438) (width 0.25) (layer "F.Cu") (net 6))
 (via (at 138.5582 105.7438) (size 0.8) (drill 0.4) (layers "F.Cu" "B.Cu") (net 6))
 (segment (start 136.9762 104.1618) (end 136.9762 102.7637) (width 0.25) (layer "B.Cu") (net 6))
 (segment (start 138.5582 105.9832) (end 138.5582 105.7438) (width 0.25) (layer "B.Cu") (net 6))
 (segment (start 136.9762 102.7637) (end 136.2125 102) (width 0.25) (layer "B.Cu") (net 6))
 (segment (start 139.075 106.5) (end 138.5582 105.9832) (width 0.25) (layer "B.Cu") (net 6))
 (segment (start 138.5582 105.7438) (end 136.9762 104.1618) (width 0.25) (layer "B.Cu") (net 6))
 (segment (start 131.4582 107.8573) (end 131.125 108.1905) (width 0.25) (layer "F.Cu") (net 5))
 (segment (start 131.125 108.1905) (end 131.125 108.7422) (width 0.25) (layer "F.Cu") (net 5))
 (segment (start 135.0261 107.8573) (end 131.4582 107.8573) (width 0.25) (layer "F.Cu") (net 5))
 (segment (start 135.6132 107.2702) (end 135.0261 107.8573) (width 0.25) (layer "F.Cu") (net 5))
 (via (at 135.6132 107.2702) (size 0.8) (drill 0.4) (layers "F.Cu" "B.Cu") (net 5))
 (segment (start 137.975 107.5) (end 137.2247 107.5) (width 0.25) (layer "B.Cu") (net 5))
 (segment (start 136.5395 106.8148) (end 136.0795 106.8148) (width 0.25) (layer "B.Cu") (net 5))
 (segment (start 136.0686 106.8148) (end 135.6132 107.2702) (width 0.25) (layer "B.Cu") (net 5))
 (segment (start 136.0795 106.8148) (end 136.0686 106.8148) (width 0.25) (layer "B.Cu") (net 5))
 (segment (start 137.2247 107.5) (end 136.5395 106.8148) (width 0.25) (layer "B.Cu") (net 5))
 (segment (start 136.2125 103.5) (end 136.0795 103.633) (width 0.25) (layer "B.Cu") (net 5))
 (segment (start 136.0795 103.633) (end 136.0795 106.8148) (width 0.25) (layer "B.Cu") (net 5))
 (segment (start 140.6127 105.239) (end 136.2786 109.5731) (width 0.25) (layer "F.Cu") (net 4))
 (segment (start 130.375 108.7422) (end 130.375 109.5731) (width 0.25) (layer "F.Cu") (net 4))
 (segment (start 136.2786 109.5731) (end 130.375 109.5731) (width 0.25) (layer "F.Cu") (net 4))
 (via (at 140.6127 105.239) (size 0.8) (drill 0.4) (layers "F.Cu" "B.Cu") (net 4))
 (segment (start 140.7875 103.5) (end 140.7875 105.0642) (width 0.25) (layer "B.Cu") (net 4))
 (segment (start 140.7875 105.0642) (end 140.6127 105.239) (width 0.25) (layer "B.Cu") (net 4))
 (segment (start 142.2125 103.5) (end 140.7875 103.5) (width 0.25) (layer "B.Cu") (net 4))
 (segment (start 130.7444 107.9113) (end 128.125 107.9113) (width 0.25) (layer "F.Cu") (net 1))
 (segment (start 132.0338 107.4069) (end 131.2488 107.4069) (width 0.25) (layer "F.Cu") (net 1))
 (segment (start 133.6029 105.8378) (end 132.0338 107.4069) (width 0.25) (layer "F.Cu") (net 1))
 (segment (start 128.125 108.7422) (end 128.125 107.9113) (width 0.25) (layer "F.Cu") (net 1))
 (segment (start 131.2488 107.4069) (end 130.7444 107.9113) (width 0.25) (layer "F.Cu") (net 1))
 (via (at 133.6029 105.8378) (size 0.8) (drill 0.4) (layers "F.Cu" "B.Cu") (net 1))
 (segment (start 142.2125 102) (end 140.7875 102) (width 0.25) (layer "B.Cu") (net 1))
 (segment (start 139.9725 101.185) (end 135.7146 101.185) (width 0.25) (layer "B.Cu") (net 1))
 (segment (start 135.4488 101.4508) (end 135.4488 103.9919) (width 0.25) (layer "B.Cu") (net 1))
 (segment (start 140.7875 102) (end 139.9725 101.185) (width 0.25) (layer "B.Cu") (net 1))
 (segment (start 135.7146 101.185) (end 135.4488 101.4508) (width 0.25) (layer "B.Cu") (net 1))
 (segment (start 135.4488 103.9919) (end 133.6029 105.8378) (width 0.25) (layer "B.Cu") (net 1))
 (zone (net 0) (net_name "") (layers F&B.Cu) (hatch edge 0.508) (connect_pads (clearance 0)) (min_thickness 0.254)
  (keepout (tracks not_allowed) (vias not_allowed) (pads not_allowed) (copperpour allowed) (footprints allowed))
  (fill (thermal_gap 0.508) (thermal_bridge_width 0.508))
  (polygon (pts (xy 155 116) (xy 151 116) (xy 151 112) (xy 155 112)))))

